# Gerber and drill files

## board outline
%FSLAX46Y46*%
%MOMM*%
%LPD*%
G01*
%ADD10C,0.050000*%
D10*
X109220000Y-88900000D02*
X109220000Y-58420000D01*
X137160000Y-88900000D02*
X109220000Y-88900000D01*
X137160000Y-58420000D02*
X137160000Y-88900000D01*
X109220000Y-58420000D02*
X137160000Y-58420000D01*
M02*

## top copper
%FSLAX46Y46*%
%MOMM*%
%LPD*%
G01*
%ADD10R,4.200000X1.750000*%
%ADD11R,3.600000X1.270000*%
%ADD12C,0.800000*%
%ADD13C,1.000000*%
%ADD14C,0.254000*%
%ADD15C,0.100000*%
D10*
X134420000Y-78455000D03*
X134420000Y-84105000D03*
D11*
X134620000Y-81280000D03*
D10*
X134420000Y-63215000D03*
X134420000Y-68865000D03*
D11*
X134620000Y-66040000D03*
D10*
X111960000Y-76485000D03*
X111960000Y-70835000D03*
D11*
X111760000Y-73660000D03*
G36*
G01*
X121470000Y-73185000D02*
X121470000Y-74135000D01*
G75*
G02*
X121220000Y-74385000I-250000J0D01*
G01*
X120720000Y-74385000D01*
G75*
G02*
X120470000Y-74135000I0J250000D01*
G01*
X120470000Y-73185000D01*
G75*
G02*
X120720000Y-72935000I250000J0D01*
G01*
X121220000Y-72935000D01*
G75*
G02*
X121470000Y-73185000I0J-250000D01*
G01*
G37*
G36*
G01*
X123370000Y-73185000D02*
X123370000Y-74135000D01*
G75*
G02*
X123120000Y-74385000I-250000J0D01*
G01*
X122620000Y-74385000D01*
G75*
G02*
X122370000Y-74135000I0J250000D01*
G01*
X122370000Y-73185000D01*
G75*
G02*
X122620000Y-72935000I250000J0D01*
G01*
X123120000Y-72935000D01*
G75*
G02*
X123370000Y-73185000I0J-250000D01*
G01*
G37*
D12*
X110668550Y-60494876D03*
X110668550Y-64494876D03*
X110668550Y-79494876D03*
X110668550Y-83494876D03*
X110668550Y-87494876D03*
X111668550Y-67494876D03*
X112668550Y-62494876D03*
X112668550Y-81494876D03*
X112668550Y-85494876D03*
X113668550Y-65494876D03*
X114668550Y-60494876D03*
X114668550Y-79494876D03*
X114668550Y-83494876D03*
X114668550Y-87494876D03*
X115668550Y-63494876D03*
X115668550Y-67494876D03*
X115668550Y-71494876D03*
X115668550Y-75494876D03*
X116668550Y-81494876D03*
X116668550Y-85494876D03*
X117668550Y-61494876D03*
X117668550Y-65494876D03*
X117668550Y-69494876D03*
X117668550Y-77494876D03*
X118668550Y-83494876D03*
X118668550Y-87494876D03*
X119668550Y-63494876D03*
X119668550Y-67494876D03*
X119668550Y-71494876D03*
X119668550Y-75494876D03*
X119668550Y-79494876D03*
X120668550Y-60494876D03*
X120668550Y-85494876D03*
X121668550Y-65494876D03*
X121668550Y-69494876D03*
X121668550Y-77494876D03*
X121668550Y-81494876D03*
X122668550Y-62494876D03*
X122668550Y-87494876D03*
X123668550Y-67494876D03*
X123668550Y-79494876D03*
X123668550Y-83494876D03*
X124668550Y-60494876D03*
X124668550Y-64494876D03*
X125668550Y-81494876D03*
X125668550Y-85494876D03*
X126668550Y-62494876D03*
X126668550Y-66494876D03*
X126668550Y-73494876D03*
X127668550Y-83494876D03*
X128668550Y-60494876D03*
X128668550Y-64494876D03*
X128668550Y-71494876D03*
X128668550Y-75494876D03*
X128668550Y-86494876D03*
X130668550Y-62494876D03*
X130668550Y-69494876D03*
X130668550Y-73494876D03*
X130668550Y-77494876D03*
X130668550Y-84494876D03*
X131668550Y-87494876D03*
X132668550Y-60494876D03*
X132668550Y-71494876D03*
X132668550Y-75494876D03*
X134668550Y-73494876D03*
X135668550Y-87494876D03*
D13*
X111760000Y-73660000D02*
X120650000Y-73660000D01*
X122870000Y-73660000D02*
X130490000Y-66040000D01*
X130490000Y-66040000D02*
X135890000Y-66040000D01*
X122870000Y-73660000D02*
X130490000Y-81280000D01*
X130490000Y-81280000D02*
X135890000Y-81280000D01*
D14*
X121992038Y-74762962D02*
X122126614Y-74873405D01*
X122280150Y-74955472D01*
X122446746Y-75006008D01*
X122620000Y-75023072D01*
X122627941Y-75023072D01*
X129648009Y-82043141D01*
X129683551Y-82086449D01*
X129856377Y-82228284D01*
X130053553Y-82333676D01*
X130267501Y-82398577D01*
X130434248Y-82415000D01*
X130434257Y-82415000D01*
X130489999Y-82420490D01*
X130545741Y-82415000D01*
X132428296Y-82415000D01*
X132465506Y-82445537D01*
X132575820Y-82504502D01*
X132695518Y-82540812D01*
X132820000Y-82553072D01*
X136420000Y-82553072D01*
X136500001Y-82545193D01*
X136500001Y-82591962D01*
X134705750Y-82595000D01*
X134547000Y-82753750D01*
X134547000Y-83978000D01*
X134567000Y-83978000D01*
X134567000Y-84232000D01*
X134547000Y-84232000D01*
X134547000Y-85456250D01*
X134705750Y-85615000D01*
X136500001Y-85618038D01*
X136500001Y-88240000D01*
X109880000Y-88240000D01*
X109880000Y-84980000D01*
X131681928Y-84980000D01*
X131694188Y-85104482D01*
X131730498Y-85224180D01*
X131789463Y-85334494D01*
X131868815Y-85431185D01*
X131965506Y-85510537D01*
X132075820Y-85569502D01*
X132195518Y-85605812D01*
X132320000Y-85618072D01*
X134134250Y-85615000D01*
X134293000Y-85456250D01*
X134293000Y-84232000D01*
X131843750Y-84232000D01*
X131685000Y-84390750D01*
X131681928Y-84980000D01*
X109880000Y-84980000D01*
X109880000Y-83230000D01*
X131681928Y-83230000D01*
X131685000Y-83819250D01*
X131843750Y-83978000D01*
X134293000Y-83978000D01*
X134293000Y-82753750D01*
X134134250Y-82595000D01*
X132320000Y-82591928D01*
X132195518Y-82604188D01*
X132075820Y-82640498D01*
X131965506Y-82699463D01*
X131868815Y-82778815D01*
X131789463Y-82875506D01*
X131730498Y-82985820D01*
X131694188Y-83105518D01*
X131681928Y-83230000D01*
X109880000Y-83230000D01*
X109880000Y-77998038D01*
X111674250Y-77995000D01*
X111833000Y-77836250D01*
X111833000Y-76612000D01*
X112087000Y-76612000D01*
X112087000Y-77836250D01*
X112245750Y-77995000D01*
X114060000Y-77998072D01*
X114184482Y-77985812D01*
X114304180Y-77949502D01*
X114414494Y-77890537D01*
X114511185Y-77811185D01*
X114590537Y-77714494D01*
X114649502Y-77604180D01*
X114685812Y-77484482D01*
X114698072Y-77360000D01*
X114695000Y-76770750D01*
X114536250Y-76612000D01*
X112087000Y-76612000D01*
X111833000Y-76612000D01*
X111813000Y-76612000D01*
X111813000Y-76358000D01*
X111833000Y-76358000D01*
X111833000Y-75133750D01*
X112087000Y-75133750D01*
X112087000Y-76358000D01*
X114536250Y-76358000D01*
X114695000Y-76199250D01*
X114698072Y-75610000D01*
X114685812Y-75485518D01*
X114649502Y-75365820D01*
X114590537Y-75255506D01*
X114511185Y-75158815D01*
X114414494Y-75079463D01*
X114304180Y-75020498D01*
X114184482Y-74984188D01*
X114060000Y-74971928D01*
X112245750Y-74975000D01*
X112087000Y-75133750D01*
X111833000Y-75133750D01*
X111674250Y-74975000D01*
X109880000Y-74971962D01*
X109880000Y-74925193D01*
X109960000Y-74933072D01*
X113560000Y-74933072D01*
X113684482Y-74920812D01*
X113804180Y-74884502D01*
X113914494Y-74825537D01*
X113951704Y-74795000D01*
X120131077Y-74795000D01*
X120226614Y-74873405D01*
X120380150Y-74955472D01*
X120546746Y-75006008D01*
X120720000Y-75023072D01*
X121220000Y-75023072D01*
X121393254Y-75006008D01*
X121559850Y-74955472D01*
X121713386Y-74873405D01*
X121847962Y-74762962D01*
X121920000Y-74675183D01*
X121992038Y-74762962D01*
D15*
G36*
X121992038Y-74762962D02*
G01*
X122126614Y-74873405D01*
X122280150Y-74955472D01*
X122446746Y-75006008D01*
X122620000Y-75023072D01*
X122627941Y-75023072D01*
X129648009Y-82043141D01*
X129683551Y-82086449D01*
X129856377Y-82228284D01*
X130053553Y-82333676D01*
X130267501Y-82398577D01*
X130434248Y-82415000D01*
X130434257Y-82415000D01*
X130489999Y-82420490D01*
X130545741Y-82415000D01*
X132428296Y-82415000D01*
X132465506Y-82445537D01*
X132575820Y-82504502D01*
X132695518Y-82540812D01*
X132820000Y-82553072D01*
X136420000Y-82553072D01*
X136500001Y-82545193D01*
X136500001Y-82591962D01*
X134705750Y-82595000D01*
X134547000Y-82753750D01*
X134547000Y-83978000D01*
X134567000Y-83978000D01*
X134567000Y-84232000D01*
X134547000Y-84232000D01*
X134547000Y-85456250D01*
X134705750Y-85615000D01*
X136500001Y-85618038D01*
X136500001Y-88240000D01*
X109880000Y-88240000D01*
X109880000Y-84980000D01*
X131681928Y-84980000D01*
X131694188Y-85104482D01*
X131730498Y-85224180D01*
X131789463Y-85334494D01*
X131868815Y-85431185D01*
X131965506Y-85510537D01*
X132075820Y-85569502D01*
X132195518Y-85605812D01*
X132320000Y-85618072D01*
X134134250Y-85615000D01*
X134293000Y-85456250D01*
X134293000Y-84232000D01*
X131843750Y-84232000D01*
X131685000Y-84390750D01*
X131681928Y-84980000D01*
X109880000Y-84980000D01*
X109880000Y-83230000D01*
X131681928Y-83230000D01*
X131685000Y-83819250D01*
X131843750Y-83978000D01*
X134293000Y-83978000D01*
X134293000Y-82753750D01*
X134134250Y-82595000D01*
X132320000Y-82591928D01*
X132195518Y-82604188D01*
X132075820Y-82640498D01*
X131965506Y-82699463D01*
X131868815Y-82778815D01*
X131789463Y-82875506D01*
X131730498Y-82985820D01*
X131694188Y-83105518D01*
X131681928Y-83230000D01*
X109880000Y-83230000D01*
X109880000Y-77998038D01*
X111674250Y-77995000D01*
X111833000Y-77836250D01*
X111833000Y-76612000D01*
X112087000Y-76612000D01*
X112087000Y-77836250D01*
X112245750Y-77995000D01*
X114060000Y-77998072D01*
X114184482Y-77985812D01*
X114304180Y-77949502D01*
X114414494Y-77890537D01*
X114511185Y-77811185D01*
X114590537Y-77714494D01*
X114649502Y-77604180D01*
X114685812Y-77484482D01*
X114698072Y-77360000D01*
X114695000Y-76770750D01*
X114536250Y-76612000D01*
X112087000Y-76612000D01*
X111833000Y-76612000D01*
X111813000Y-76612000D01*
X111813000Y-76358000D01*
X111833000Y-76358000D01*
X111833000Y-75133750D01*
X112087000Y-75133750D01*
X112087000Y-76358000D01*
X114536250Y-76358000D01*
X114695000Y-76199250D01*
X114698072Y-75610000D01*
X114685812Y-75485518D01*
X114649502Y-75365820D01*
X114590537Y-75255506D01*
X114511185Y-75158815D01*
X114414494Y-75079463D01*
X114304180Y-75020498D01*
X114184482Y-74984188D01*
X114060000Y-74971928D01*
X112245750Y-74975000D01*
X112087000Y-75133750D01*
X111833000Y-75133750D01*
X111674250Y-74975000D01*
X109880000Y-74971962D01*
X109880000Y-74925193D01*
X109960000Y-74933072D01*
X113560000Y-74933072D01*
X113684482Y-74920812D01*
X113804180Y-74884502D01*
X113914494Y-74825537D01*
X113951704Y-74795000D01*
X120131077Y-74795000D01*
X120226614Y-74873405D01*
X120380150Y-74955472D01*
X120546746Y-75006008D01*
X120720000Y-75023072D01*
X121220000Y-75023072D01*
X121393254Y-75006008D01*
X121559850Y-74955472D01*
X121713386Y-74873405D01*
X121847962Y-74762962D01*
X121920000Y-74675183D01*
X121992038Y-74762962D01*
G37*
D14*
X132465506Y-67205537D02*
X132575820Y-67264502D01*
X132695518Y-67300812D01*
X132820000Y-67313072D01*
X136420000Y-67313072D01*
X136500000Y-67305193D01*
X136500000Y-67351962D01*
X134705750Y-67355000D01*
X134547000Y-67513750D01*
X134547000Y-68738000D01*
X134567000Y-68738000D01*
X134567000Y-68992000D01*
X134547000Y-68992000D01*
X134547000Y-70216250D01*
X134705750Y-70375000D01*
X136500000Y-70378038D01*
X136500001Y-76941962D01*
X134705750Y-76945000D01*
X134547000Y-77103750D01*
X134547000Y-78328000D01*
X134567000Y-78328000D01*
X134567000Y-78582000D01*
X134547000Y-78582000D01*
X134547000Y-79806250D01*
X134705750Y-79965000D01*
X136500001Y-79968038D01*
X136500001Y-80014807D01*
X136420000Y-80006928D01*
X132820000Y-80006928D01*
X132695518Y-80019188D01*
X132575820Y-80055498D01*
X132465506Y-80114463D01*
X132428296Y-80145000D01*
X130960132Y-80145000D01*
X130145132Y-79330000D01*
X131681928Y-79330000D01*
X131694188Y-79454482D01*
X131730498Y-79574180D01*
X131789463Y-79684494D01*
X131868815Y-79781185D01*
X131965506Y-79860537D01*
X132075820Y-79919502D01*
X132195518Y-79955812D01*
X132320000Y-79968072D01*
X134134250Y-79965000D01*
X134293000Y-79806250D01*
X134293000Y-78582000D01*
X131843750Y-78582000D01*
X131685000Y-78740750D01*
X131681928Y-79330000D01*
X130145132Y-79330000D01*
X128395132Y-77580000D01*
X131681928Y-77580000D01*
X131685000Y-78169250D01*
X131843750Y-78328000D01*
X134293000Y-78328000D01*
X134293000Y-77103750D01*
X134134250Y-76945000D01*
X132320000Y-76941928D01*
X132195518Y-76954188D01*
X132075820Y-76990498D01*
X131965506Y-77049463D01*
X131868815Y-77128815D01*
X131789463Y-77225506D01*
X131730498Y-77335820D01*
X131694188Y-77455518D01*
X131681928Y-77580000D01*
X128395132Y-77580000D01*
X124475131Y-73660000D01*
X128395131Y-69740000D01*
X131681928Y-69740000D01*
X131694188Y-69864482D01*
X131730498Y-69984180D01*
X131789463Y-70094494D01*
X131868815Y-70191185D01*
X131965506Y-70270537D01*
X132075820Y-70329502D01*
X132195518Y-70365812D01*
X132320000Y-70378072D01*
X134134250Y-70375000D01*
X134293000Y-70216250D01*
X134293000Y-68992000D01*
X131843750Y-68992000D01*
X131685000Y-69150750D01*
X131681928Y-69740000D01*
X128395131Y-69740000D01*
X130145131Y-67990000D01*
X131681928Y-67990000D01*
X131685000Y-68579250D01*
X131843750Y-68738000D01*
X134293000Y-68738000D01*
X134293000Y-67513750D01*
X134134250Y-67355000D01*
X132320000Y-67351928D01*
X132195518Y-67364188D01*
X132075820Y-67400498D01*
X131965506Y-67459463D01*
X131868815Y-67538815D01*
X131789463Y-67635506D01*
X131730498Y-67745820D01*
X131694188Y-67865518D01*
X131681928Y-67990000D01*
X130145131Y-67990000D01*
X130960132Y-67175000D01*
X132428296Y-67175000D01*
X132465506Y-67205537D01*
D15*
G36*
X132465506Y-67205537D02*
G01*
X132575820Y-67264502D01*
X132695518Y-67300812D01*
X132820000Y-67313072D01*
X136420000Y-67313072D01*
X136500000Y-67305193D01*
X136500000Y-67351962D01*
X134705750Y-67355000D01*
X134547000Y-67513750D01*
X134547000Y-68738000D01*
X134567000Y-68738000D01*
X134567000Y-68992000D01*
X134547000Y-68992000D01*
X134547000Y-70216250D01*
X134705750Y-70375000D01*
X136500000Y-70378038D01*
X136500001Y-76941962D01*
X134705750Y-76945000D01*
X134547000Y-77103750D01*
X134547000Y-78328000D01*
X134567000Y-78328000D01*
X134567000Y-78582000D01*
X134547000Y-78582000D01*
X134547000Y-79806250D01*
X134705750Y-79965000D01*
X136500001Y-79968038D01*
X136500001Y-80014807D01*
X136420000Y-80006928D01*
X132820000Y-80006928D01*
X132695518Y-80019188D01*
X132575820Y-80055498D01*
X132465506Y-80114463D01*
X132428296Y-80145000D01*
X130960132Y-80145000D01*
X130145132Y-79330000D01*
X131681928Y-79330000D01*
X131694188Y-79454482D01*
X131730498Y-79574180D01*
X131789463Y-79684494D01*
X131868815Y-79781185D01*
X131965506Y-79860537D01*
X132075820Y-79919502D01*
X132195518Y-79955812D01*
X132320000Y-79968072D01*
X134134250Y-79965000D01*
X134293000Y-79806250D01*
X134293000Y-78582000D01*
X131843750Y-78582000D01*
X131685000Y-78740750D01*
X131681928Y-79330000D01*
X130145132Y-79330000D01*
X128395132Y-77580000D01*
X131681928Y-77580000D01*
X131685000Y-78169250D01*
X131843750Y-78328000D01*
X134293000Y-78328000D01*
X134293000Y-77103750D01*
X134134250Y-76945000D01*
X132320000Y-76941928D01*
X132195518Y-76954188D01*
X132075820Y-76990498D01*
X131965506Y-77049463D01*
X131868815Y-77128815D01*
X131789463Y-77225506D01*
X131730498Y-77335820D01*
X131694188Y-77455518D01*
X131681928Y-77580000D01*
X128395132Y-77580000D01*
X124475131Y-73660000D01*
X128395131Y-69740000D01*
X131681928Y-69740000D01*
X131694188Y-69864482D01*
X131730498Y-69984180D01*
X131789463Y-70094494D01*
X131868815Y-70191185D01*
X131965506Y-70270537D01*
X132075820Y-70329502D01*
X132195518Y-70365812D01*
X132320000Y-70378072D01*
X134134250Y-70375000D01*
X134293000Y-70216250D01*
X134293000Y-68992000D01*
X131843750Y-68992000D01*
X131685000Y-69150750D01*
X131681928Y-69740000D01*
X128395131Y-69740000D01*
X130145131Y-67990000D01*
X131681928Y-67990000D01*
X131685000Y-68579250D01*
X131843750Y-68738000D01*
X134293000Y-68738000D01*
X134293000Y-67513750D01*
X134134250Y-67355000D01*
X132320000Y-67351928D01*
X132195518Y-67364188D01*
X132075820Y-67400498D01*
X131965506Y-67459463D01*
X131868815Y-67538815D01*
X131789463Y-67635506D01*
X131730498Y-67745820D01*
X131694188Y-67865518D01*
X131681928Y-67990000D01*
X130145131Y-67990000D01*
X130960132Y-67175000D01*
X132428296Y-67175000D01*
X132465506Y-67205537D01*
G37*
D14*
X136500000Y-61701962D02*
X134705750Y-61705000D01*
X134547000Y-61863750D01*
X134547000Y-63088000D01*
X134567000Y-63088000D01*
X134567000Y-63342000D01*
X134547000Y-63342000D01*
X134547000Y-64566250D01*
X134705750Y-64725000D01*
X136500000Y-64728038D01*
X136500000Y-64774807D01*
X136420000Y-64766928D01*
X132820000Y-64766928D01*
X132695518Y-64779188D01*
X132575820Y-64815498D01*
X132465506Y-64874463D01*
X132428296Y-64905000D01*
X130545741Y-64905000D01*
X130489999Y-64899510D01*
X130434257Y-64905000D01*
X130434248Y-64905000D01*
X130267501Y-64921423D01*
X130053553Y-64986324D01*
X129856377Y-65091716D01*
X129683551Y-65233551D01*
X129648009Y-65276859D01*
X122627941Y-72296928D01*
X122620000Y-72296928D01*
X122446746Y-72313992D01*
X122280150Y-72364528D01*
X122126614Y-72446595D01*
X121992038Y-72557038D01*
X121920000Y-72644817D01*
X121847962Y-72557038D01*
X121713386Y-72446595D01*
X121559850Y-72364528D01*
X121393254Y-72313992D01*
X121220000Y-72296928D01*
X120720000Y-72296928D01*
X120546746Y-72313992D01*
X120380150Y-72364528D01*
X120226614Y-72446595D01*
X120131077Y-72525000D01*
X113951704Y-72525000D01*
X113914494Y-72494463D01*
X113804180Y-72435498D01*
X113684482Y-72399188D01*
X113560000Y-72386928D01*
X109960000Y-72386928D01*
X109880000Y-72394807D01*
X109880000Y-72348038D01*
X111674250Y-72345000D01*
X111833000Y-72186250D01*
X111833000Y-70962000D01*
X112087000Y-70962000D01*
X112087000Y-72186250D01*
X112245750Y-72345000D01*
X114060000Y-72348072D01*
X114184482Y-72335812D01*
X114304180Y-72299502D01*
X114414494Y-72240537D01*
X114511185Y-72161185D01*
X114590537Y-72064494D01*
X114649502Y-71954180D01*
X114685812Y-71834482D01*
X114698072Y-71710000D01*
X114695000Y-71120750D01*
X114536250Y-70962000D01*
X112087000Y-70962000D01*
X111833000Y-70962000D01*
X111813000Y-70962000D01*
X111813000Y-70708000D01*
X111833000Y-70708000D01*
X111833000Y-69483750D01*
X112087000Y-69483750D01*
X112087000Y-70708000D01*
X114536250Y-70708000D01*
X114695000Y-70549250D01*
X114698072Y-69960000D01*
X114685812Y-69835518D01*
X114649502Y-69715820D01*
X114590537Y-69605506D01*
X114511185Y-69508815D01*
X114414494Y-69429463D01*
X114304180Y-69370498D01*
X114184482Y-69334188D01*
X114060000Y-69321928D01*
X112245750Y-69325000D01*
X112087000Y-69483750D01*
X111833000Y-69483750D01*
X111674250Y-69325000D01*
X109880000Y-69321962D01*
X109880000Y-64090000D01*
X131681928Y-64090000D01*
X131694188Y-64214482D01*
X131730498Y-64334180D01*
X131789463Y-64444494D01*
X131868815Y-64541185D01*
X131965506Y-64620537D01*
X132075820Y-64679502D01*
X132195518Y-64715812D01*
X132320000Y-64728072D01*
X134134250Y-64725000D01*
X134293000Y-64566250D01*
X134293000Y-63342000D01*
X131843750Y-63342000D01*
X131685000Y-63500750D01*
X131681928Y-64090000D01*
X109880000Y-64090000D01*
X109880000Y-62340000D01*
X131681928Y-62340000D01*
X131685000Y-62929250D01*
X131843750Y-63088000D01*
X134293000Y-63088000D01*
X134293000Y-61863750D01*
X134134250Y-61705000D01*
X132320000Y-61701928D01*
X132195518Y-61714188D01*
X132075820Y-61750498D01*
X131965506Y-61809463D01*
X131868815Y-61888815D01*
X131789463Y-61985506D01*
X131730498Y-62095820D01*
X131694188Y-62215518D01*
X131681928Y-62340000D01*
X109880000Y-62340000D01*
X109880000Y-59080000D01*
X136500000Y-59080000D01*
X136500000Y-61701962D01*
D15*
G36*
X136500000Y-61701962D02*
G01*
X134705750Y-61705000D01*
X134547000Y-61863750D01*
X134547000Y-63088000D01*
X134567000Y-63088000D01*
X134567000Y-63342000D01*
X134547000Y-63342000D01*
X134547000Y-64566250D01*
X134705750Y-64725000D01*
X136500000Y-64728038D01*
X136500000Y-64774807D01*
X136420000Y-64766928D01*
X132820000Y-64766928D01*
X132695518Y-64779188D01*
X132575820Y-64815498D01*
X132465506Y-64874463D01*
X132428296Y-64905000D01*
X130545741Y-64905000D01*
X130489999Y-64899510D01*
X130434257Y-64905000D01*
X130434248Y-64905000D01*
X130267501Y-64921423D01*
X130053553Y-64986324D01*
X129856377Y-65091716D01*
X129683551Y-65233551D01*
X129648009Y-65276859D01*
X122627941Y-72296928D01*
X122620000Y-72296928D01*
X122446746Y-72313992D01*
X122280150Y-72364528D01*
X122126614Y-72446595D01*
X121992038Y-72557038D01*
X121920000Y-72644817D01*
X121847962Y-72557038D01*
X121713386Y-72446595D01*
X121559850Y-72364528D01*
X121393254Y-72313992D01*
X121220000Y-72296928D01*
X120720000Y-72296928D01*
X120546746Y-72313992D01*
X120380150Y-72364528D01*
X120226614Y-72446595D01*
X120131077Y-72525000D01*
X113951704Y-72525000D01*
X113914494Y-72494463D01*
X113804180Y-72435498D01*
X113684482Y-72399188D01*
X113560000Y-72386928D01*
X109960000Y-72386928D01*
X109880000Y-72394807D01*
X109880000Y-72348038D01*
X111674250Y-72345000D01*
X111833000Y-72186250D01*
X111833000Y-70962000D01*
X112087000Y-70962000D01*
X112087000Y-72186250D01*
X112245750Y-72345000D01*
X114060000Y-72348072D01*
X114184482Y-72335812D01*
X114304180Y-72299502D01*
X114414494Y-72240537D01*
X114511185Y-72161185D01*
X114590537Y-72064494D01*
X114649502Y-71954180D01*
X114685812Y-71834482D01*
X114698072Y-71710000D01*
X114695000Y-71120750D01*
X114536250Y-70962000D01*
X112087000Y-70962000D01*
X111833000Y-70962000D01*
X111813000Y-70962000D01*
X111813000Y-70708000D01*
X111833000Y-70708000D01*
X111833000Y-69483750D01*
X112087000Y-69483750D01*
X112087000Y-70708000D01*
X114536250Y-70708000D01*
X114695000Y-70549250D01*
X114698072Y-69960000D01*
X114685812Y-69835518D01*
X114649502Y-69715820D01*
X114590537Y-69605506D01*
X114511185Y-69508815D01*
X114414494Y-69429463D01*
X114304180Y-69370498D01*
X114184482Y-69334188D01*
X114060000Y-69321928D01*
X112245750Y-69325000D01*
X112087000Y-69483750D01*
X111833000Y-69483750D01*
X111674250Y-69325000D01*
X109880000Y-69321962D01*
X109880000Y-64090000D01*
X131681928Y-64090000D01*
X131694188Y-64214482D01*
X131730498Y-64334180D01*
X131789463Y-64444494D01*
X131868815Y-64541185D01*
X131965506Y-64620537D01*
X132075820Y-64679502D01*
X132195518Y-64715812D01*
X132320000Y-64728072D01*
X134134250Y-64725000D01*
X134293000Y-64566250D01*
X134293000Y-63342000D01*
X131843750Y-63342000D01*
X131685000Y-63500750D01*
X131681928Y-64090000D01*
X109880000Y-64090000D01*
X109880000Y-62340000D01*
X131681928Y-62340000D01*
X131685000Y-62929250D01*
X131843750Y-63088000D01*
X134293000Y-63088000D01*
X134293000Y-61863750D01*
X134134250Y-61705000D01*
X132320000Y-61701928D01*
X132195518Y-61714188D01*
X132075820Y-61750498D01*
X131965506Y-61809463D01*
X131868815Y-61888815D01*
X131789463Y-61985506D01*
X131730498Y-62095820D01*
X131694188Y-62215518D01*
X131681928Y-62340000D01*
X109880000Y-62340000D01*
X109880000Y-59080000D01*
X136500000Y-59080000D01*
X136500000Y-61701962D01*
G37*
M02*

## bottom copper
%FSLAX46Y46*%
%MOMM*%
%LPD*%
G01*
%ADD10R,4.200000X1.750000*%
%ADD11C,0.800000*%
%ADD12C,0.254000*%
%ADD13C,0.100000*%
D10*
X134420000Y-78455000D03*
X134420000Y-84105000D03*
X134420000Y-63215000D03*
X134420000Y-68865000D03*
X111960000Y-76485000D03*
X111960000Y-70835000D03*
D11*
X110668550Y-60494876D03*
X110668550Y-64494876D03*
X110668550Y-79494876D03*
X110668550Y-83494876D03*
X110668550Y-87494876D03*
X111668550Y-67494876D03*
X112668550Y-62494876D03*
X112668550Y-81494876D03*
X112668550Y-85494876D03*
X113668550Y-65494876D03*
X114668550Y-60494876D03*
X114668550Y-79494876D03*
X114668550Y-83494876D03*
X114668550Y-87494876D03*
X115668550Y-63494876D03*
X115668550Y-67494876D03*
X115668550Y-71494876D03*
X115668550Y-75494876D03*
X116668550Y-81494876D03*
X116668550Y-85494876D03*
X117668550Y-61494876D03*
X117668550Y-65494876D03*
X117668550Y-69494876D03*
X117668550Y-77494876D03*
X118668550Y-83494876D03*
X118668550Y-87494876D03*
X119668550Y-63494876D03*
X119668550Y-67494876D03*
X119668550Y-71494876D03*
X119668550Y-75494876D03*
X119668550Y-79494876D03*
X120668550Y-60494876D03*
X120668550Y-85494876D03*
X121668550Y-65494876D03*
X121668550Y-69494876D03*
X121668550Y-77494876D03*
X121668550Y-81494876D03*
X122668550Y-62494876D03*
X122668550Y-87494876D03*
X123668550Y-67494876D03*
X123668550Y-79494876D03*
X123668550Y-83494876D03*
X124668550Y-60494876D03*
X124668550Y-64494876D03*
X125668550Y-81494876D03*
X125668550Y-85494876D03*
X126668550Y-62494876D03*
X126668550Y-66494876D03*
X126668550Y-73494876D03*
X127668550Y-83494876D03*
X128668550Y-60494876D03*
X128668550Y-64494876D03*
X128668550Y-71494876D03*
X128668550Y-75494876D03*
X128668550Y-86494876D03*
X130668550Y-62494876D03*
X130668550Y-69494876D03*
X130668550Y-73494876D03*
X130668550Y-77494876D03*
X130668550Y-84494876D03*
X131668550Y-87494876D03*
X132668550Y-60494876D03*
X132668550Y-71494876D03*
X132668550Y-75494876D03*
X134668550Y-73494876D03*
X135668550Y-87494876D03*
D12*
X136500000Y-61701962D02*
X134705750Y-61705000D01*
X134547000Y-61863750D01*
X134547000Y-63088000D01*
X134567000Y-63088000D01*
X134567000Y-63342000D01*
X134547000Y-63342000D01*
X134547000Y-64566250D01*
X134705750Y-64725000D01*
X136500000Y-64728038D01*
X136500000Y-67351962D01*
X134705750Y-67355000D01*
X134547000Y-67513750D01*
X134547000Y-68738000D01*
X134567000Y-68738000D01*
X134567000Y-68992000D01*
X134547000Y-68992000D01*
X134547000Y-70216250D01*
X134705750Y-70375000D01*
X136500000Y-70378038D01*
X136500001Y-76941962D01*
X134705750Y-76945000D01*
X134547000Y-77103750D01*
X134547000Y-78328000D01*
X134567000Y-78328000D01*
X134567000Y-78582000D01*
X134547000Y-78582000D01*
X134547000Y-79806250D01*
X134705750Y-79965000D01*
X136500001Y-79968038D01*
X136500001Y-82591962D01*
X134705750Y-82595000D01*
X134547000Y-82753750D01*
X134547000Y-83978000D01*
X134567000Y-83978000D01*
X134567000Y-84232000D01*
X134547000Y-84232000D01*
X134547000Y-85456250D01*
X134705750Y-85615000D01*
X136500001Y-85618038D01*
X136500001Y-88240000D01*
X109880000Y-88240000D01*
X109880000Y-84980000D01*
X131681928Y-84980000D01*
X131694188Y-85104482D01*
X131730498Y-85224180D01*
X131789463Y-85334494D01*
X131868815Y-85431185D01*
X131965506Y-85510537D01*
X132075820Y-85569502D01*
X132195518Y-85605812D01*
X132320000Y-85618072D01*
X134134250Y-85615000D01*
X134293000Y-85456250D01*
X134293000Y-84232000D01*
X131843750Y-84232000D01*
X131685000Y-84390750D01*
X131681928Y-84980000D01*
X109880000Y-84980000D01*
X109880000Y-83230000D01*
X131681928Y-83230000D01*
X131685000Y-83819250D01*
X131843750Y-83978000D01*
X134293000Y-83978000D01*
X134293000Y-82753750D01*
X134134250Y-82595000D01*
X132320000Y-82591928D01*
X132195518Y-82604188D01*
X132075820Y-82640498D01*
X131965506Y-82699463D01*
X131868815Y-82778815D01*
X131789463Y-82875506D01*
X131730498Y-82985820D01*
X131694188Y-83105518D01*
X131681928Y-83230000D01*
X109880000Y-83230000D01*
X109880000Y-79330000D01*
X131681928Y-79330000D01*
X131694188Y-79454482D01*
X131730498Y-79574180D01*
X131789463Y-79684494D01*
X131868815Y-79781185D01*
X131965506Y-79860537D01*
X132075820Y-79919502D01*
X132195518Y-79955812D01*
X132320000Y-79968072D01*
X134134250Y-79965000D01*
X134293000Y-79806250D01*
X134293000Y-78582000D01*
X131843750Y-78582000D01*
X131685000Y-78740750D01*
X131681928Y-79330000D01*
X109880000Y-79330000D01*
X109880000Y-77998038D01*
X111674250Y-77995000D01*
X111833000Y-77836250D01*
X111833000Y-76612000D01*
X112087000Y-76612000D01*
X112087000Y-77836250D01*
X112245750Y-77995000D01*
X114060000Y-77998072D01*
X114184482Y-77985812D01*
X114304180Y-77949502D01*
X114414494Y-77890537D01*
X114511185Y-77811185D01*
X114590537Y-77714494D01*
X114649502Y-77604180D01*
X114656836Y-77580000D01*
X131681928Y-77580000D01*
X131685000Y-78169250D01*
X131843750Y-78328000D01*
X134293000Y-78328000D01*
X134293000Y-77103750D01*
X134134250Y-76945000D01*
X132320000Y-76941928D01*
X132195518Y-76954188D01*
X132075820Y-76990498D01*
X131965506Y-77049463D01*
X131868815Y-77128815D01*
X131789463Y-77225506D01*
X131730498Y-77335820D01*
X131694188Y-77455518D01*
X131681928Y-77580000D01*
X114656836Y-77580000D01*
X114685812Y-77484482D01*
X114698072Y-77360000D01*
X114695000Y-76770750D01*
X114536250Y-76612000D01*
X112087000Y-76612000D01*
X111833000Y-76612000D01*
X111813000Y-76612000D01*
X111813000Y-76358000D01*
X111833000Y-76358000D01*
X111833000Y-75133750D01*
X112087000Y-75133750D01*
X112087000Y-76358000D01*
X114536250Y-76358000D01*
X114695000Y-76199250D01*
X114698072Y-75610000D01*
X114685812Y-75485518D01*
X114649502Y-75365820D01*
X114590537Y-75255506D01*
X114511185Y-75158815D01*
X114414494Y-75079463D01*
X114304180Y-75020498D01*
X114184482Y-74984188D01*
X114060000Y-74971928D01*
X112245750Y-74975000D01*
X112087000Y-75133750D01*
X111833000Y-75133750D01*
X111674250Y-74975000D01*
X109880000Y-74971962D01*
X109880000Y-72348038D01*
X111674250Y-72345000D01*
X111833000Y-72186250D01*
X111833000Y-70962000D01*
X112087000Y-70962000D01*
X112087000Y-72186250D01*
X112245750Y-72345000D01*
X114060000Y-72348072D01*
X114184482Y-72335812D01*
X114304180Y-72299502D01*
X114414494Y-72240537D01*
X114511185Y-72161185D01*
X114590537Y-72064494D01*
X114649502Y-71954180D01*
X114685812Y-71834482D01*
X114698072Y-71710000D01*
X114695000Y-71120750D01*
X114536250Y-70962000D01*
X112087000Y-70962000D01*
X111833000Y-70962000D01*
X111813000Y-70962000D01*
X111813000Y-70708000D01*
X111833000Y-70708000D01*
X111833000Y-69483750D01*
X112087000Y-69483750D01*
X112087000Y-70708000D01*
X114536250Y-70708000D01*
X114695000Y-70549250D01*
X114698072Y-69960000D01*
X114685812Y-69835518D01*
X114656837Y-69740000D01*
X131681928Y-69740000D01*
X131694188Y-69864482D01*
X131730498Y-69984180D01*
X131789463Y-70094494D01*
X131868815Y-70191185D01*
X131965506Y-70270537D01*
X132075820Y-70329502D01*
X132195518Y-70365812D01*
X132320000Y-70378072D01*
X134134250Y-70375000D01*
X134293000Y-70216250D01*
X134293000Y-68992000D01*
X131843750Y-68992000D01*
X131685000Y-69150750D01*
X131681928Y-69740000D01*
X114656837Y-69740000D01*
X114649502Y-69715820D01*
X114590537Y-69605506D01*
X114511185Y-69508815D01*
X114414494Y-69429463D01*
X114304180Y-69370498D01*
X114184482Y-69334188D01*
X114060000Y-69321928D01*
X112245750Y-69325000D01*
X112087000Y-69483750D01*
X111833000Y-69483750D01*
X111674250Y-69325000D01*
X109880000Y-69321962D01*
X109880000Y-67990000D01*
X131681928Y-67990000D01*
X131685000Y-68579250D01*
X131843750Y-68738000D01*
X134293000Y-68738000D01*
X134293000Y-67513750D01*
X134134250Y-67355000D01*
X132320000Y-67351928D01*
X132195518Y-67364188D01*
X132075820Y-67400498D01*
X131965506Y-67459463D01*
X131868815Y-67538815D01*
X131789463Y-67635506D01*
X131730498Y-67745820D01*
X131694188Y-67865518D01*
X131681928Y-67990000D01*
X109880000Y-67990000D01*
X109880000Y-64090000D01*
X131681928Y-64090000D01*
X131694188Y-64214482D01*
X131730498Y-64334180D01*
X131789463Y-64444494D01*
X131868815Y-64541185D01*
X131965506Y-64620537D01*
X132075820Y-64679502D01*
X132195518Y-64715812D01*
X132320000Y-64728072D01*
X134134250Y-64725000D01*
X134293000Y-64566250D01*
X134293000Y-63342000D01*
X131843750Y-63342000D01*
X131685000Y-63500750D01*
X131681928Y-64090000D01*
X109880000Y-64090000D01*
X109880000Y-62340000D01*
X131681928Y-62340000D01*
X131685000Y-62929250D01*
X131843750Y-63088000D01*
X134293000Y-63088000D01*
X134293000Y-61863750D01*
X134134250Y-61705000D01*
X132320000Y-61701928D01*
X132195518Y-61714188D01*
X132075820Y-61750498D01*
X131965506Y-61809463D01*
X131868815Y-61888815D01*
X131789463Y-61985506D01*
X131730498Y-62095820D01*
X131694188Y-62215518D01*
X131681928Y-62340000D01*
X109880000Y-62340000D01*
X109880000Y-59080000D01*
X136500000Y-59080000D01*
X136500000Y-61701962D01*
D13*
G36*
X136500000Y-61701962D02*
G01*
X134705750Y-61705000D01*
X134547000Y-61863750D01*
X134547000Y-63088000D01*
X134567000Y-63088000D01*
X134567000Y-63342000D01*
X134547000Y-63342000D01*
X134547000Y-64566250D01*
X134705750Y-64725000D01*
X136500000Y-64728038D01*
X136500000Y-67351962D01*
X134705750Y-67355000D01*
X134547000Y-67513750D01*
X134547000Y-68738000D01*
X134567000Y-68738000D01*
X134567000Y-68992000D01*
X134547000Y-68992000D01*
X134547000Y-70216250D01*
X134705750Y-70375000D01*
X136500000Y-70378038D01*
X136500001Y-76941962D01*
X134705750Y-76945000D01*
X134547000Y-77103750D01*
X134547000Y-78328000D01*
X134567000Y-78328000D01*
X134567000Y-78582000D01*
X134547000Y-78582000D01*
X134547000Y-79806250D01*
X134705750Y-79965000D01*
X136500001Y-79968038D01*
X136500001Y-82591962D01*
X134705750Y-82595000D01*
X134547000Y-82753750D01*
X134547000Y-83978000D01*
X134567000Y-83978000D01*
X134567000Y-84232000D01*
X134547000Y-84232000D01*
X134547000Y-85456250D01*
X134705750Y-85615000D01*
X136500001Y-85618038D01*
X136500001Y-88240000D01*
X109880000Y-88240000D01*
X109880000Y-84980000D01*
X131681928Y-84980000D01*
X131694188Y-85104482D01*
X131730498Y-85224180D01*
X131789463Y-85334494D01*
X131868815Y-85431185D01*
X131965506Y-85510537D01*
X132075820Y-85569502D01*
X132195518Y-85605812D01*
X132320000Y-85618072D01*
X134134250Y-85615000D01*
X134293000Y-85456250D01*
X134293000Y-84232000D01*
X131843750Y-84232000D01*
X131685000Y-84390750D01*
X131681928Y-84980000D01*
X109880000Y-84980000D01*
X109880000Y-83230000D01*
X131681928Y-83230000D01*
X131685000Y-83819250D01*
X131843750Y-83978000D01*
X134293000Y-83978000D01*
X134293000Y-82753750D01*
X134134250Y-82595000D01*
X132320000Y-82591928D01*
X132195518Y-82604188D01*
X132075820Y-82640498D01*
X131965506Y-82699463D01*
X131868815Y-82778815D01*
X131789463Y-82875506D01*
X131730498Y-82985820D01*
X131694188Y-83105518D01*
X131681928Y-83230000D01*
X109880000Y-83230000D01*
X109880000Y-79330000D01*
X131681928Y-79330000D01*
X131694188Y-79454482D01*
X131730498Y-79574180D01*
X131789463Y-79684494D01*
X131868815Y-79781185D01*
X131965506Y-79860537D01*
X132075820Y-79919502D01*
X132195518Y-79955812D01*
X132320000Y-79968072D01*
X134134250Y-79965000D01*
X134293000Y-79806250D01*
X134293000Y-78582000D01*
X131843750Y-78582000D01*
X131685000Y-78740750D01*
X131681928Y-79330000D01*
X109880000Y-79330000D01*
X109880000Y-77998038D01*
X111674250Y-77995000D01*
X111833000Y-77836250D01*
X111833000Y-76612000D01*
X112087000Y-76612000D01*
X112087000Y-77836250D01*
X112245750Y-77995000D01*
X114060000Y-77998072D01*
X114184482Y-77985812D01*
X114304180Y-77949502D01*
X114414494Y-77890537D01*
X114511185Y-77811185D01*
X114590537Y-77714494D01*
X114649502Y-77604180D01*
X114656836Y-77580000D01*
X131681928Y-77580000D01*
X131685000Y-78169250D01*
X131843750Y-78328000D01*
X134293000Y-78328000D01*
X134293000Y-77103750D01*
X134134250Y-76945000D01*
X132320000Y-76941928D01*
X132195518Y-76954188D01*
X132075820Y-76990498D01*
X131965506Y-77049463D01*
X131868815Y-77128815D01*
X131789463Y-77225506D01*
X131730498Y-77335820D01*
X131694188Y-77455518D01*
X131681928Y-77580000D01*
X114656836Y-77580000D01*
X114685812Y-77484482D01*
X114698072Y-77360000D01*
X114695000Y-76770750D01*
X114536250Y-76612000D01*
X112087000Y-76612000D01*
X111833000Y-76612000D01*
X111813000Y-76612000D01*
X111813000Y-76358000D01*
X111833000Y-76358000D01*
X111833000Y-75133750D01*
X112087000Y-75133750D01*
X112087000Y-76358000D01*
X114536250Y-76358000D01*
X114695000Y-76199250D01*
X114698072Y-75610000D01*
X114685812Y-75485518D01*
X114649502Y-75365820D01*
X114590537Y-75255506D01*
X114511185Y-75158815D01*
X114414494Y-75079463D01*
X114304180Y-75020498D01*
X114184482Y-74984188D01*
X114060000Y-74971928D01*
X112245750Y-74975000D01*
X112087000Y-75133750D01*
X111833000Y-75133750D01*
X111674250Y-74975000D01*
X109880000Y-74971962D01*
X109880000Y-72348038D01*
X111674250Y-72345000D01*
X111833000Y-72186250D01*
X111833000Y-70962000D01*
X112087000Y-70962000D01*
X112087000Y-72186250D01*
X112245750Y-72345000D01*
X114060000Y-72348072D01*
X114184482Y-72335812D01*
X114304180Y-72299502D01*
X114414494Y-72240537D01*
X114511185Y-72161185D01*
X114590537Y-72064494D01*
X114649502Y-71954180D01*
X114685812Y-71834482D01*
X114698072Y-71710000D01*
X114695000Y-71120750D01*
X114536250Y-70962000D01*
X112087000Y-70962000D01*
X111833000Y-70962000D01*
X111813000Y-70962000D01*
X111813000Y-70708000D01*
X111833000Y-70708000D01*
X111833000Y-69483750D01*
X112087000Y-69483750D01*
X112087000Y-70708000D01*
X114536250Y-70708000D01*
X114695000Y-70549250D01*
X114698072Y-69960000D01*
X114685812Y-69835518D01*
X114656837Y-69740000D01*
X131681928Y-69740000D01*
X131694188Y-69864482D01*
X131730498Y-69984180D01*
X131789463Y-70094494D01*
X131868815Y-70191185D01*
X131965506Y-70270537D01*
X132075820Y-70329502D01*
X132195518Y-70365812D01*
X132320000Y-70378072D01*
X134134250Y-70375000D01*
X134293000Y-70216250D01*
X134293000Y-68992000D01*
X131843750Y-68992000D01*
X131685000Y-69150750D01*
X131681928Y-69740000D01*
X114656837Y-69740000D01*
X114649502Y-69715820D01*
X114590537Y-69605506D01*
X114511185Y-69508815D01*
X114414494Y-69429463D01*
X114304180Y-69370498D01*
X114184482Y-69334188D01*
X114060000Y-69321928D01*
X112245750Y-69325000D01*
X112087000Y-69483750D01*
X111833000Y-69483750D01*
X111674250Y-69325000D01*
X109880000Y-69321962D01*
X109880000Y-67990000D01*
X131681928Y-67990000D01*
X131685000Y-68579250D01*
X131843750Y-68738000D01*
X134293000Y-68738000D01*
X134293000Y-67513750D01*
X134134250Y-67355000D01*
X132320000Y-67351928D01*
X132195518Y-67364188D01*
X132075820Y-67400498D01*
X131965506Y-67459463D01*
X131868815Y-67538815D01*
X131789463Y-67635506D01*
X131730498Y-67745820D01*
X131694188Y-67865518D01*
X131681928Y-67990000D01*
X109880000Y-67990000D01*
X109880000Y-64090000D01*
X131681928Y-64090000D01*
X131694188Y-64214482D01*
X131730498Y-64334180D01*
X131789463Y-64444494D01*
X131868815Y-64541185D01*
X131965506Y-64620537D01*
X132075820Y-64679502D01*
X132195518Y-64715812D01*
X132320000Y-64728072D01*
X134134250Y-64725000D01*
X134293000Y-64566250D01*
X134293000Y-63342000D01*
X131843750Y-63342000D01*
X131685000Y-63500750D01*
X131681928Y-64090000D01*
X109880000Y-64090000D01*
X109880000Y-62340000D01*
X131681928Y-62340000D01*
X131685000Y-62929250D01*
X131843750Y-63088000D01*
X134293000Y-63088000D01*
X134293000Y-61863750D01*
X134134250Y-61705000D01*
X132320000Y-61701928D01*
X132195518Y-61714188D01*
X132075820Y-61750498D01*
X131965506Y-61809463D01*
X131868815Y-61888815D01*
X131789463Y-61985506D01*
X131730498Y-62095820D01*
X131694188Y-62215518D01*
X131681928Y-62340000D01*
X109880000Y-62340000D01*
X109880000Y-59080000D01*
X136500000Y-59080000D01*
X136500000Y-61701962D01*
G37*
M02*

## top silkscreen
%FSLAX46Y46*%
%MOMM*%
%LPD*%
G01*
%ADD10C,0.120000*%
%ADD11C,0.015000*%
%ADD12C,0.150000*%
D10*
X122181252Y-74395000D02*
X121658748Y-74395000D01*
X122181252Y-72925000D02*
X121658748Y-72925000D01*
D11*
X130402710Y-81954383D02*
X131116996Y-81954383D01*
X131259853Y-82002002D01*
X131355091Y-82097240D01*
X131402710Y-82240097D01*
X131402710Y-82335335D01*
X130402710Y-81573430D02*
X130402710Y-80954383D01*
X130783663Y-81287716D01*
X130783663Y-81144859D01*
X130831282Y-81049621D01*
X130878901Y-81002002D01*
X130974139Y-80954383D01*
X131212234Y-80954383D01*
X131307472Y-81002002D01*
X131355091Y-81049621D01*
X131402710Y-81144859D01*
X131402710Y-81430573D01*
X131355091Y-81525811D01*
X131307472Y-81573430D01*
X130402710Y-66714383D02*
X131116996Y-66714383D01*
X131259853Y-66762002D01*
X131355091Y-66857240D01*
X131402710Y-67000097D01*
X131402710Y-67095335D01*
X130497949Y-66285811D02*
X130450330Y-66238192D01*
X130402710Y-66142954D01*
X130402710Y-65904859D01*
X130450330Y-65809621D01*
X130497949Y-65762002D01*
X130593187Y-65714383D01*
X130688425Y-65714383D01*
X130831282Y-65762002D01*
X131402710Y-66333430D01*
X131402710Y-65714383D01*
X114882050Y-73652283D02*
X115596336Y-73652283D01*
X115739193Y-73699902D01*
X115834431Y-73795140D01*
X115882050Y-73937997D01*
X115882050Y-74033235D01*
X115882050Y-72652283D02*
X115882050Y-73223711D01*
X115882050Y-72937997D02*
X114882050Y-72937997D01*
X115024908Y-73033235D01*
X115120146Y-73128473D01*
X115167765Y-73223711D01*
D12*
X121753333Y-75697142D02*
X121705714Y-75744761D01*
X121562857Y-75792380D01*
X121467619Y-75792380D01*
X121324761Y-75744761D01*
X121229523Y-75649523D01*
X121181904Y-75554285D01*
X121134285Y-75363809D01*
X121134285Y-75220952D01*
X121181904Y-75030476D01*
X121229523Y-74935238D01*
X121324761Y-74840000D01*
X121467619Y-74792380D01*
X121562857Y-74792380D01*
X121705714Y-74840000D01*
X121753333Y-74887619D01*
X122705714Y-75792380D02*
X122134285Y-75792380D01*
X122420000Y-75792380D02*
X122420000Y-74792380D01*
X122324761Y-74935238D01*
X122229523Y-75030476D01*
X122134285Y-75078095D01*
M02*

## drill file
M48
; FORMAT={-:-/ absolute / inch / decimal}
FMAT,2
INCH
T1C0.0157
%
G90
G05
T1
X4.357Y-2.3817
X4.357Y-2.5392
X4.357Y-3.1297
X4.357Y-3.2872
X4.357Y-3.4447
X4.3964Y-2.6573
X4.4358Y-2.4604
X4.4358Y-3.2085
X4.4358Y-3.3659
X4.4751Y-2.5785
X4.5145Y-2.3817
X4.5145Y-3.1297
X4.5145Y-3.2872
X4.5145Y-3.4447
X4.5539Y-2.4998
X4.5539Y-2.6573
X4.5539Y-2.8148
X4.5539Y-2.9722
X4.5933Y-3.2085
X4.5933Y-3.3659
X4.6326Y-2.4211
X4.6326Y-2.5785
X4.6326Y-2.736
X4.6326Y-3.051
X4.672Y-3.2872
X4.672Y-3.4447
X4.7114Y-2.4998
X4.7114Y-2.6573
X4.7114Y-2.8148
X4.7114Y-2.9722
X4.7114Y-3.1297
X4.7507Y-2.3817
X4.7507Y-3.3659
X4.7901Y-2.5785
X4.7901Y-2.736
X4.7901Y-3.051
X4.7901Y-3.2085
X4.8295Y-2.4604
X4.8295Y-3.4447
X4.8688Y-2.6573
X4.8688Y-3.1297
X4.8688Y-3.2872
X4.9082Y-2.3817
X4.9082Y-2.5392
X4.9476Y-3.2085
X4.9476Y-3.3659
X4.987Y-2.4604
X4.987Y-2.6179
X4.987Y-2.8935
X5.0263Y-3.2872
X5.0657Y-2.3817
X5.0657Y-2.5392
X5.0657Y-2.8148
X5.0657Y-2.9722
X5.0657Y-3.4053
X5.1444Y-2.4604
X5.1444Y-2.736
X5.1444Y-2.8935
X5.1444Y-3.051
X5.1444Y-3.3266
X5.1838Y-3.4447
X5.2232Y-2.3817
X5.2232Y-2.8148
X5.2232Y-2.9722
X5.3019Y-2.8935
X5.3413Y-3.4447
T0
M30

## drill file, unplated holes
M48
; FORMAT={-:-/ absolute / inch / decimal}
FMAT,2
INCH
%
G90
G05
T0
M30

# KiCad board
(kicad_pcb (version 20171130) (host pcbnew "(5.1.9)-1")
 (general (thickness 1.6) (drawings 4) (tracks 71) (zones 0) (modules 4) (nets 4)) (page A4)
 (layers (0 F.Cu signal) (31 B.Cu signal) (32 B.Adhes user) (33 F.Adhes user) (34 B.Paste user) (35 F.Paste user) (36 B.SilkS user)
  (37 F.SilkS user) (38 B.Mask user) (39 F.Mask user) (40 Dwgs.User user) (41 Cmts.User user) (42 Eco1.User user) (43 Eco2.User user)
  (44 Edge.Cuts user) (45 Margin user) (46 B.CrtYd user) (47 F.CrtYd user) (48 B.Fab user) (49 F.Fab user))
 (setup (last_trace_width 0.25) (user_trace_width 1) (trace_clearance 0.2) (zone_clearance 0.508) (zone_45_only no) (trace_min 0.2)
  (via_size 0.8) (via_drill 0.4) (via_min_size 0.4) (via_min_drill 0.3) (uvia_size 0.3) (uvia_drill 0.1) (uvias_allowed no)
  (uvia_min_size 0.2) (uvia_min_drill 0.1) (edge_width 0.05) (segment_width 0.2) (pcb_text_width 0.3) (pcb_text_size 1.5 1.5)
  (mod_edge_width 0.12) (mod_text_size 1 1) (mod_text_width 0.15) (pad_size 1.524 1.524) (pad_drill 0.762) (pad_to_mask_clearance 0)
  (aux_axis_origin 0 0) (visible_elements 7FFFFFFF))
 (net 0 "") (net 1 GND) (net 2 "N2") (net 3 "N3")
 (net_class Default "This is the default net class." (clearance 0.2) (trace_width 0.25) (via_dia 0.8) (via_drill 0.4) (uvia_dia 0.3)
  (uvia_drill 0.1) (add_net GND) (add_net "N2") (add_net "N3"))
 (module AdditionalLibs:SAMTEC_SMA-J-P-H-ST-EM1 (layer F.Cu) (at 134.62 81.28 90)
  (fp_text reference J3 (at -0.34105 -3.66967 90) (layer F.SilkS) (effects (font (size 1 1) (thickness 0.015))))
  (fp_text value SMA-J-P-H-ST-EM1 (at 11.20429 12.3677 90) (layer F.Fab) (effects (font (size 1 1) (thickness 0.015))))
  (pad 3_2 smd rect (at 2.825 -0.2 90) (size 1.75 4.2) (layers B.Cu B.Paste B.Mask) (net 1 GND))
  (pad 2_2 smd rect (at -2.825 -0.2 90) (size 1.75 4.2) (layers B.Cu B.Paste B.Mask) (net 1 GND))
  (pad 3_1 smd rect (at 2.825 -0.2 90) (size 1.75 4.2) (layers F.Cu F.Paste F.Mask) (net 1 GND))
  (pad 2_1 smd rect (at -2.825 -0.2 90) (size 1.75 4.2) (layers F.Cu F.Paste F.Mask) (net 1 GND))
  (pad 1 smd rect (at 0 0 90) (size 1.27 3.6) (layers F.Cu F.Paste F.Mask) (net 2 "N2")))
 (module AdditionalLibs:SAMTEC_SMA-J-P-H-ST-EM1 (layer F.Cu) (at 134.62 66.04 90)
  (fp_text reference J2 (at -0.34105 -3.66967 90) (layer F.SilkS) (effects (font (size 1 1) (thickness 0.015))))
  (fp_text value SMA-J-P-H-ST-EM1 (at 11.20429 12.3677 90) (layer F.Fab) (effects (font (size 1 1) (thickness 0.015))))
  (pad 3_2 smd rect (at 2.825 -0.2 90) (size 1.75 4.2) (layers B.Cu B.Paste B.Mask) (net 1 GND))
  (pad 2_2 smd rect (at -2.825 -0.2 90) (size 1.75 4.2) (layers B.Cu B.Paste B.Mask) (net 1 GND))
  (pad 3_1 smd rect (at 2.825 -0.2 90) (size 1.75 4.2) (layers F.Cu F.Paste F.Mask) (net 1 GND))
  (pad 2_1 smd rect (at -2.825 -0.2 90) (size 1.75 4.2) (layers F.Cu F.Paste F.Mask) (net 1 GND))
  (pad 1 smd rect (at 0 0 90) (size 1.27 3.6) (layers F.Cu F.Paste F.Mask) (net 2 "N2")))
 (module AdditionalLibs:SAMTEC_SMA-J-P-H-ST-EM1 (layer F.Cu) (at 111.76 73.66 270)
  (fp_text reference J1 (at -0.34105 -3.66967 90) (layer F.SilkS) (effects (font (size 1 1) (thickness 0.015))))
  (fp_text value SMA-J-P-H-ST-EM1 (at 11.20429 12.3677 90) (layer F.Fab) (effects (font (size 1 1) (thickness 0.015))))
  (pad 3_2 smd rect (at 2.825 -0.2 270) (size 1.75 4.2) (layers B.Cu B.Paste B.Mask) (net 1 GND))
  (pad 2_2 smd rect (at -2.825 -0.2 270) (size 1.75 4.2) (layers B.Cu B.Paste B.Mask) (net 1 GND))
  (pad 3_1 smd rect (at 2.825 -0.2 270) (size 1.75 4.2) (layers F.Cu F.Paste F.Mask) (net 1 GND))
  (pad 2_1 smd rect (at -2.825 -0.2 270) (size 1.75 4.2) (layers F.Cu F.Paste F.Mask) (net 1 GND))
  (pad 1 smd rect (at 0 0 270) (size 1.27 3.6) (layers F.Cu F.Paste F.Mask) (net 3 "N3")))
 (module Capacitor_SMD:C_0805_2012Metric (layer F.Cu) (at 121.92 73.66 180)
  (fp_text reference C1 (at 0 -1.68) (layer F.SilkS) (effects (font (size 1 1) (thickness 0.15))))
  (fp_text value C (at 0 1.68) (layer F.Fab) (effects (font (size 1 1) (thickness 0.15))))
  (fp_line (start -0.261252 -0.735) (end 0.261252 -0.735) (layer F.SilkS) (width 0.12))
  (fp_line (start -0.261252 0.735) (end 0.261252 0.735) (layer F.SilkS) (width 0.12))
  (pad 2 smd roundrect (at 0.95 0 180) (size 1 1.45) (layers F.Cu F.Paste F.Mask) (roundrect_rratio 0.25) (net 3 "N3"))
  (pad 1 smd roundrect (at -0.95 0 180) (size 1 1.45) (layers F.Cu F.Paste F.Mask) (roundrect_rratio 0.25) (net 2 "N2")))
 (gr_line (start 109.22 88.9) (end 109.22 58.42) (layer Edge.Cuts) (width 0.05))
 (gr_line (start 137.16 88.9) (end 109.22 88.9) (layer Edge.Cuts) (width 0.05))
 (gr_line (start 137.16 58.42) (end 137.16 88.9) (layer Edge.Cuts) (width 0.05))
 (gr_line (start 109.22 58.42) (end 137.16 58.42) (layer Edge.Cuts) (width 0.05))
 (via (at 110.66855 60.494876) (size 0.8) (drill 0.4) (layers F.Cu B.Cu) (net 1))
 (via (at 110.66855 64.494876) (size 0.8) (drill 0.4) (layers F.Cu B.Cu) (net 1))
 (via (at 110.66855 79.494876) (size 0.8) (drill 0.4) (layers F.Cu B.Cu) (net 1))
 (via (at 110.66855 83.494876) (size 0.8) (drill 0.4) (layers F.Cu B.Cu) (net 1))
 (via (at 110.66855 87.494876) (size 0.8) (drill 0.4) (layers F.Cu B.Cu) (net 1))
 (via (at 111.66855 67.494876) (size 0.8) (drill 0.4) (layers F.Cu B.Cu) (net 1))
 (via (at 112.66855 62.494876) (size 0.8) (drill 0.4) (layers F.Cu B.Cu) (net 1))
 (via (at 112.66855 81.494876) (size 0.8) (drill 0.4) (layers F.Cu B.Cu) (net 1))
 (via (at 112.66855 85.494876) (size 0.8) (drill 0.4) (layers F.Cu B.Cu) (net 1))
 (via (at 113.66855 65.494876) (size 0.8) (drill 0.4) (layers F.Cu B.Cu) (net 1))
 (via (at 114.66855 60.494876) (size 0.8) (drill 0.4) (layers F.Cu B.Cu) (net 1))
 (via (at 114.66855 79.494876) (size 0.8) (drill 0.4) (layers F.Cu B.Cu) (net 1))
 (via (at 114.66855 83.494876) (size 0.8) (drill 0.4) (layers F.Cu B.Cu) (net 1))
 (via (at 114.66855 87.494876) (size 0.8) (drill 0.4) (layers F.Cu B.Cu) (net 1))
 (via (at 115.66855 63.494876) (size 0.8) (drill 0.4) (layers F.Cu B.Cu) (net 1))
 (via (at 115.66855 67.494876) (size 0.8) (drill 0.4) (layers F.Cu B.Cu) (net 1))
 (via (at 115.66855 71.494876) (size 0.8) (drill 0.4) (layers F.Cu B.Cu) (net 1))
 (via (at 115.66855 75.494876) (size 0.8) (drill 0.4) (layers F.Cu B.Cu) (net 1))
 (via (at 116.66855 81.494876) (size 0.8) (drill 0.4) (layers F.Cu B.Cu) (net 1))
 (via (at 116.66855 85.494876) (size 0.8) (drill 0.4) (layers F.Cu B.Cu) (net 1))
 (via (at 117.66855 61.494876) (size 0.8) (drill 0.4) (layers F.Cu B.Cu) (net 1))
 (via (at 117.66855 65.494876) (size 0.8) (drill 0.4) (layers F.Cu B.Cu) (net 1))
 (via (at 117.66855 69.494876) (size 0.8) (drill 0.4) (layers F.Cu B.Cu) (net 1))
 (via (at 117.66855 77.494876) (size 0.8) (drill 0.4) (layers F.Cu B.Cu) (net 1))
 (via (at 118.66855 83.494876) (size 0.8) (drill 0.4) (layers F.Cu B.Cu) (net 1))
 (via (at 118.66855 87.494876) (size 0.8) (drill 0.4) (layers F.Cu B.Cu) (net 1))
 (via (at 119.66855 63.494876) (size 0.8) (drill 0.4) (layers F.Cu B.Cu) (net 1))
 (via (at 119.66855 67.494876) (size 0.8) (drill 0.4) (layers F.Cu B.Cu) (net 1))
 (via (at 119.66855 71.494876) (size 0.8) (drill 0.4) (layers F.Cu B.Cu) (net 1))
 (via (at 119.66855 75.494876) (size 0.8) (drill 0.4) (layers F.Cu B.Cu) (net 1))
 (via (at 119.66855 79.494876) (size 0.8) (drill 0.4) (layers F.Cu B.Cu) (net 1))
 (via (at 120.66855 60.494876) (size 0.8) (drill 0.4) (layers F.Cu B.Cu) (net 1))
 (via (at 120.66855 85.494876) (size 0.8) (drill 0.4) (layers F.Cu B.Cu) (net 1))
 (via (at 121.66855 65.494876) (size 0.8) (drill 0.4) (layers F.Cu B.Cu) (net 1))
 (via (at 121.66855 69.494876) (size 0.8) (drill 0.4) (layers F.Cu B.Cu) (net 1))
 (via (at 121.66855 77.494876) (size 0.8) (drill 0.4) (layers F.Cu B.Cu) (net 1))
 (via (at 121.66855 81.494876) (size 0.8) (drill 0.4) (layers F.Cu B.Cu) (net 1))
 (via (at 122.66855 62.494876) (size 0.8) (drill 0.4) (layers F.Cu B.Cu) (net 1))
 (via (at 122.66855 87.494876) (size 0.8) (drill 0.4) (layers F.Cu B.Cu) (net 1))
 (via (at 123.66855 67.494876) (size 0.8) (drill 0.4) (layers F.Cu B.Cu) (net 1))
 (via (at 123.66855 79.494876) (size 0.8) (drill 0.4) (layers F.Cu B.Cu) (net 1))
 (via (at 123.66855 83.494876) (size 0.8) (drill 0.4) (layers F.Cu B.Cu) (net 1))
 (via (at 124.66855 60.494876) (size 0.8) (drill 0.4) (layers F.Cu B.Cu) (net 1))
 (via (at 124.66855 64.494876) (size 0.8) (drill 0.4) (layers F.Cu B.Cu) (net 1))
 (via (at 125.66855 81.494876) (size 0.8) (drill 0.4) (layers F.Cu B.Cu) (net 1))
 (via (at 125.66855 85.494876) (size 0.8) (drill 0.4) (layers F.Cu B.Cu) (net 1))
 (via (at 126.66855 62.494876) (size 0.8) (drill 0.4) (layers F.Cu B.Cu) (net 1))
 (via (at 126.66855 66.494876) (size 0.8) (drill 0.4) (layers F.Cu B.Cu) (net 1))
 (via (at 126.66855 73.494876) (size 0.8) (drill 0.4) (layers F.Cu B.Cu) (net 1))
 (via (at 127.66855 83.494876) (size 0.8) (drill 0.4) (layers F.Cu B.Cu) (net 1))
 (via (at 128.66855 60.494876) (size 0.8) (drill 0.4) (layers F.Cu B.Cu) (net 1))
 (via (at 128.66855 64.494876) (size 0.8) (drill 0.4) (layers F.Cu B.Cu) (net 1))
 (via (at 128.66855 71.494876) (size 0.8) (drill 0.4) (layers F.Cu B.Cu) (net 1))
 (via (at 128.66855 75.494876) (size 0.8) (drill 0.4) (layers F.Cu B.Cu) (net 1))
 (via (at 128.66855 86.494876) (size 0.8) (drill 0.4) (layers F.Cu B.Cu) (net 1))
 (via (at 130.66855 62.494876) (size 0.8) (drill 0.4) (layers F.Cu B.Cu) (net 1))
 (via (at 130.66855 69.494876) (size 0.8) (drill 0.4) (layers F.Cu B.Cu) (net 1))
 (via (at 130.66855 73.494876) (size 0.8) (drill 0.4) (layers F.Cu B.Cu) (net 1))
 (via (at 130.66855 77.494876) (size 0.8) (drill 0.4) (layers F.Cu B.Cu) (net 1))
 (via (at 130.66855 84.494876) (size 0.8) (drill 0.4) (layers F.Cu B.Cu) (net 1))
 (via (at 131.66855 87.494876) (size 0.8) (drill 0.4) (layers F.Cu B.Cu) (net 1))
 (via (at 132.66855 60.494876) (size 0.8) (drill 0.4) (layers F.Cu B.Cu) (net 1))
 (via (at 132.66855 71.494876) (size 0.8) (drill 0.4) (layers F.Cu B.Cu) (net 1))
 (via (at 132.66855 75.494876) (size 0.8) (drill 0.4) (layers F.Cu B.Cu) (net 1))
 (via (at 134.66855 73.494876) (size 0.8) (drill 0.4) (layers F.Cu B.Cu) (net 1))
 (via (at 135.66855 87.494876) (size 0.8) (drill 0.4) (layers F.Cu B.Cu) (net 1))
 (segment (start 111.76 73.66) (end 120.65 73.66) (width 1) (layer F.Cu) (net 3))
 (segment (start 122.87 73.66) (end 130.49 66.04) (width 1) (layer F.Cu) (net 2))
 (segment (start 130.49 66.04) (end 135.89 66.04) (width 1) (layer F.Cu) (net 2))
 (segment (start 122.87 73.66) (end 130.49 81.28) (width 1) (layer F.Cu) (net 2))
 (segment (start 130.49 81.28) (end 135.89 81.28) (width 1) (layer F.Cu) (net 2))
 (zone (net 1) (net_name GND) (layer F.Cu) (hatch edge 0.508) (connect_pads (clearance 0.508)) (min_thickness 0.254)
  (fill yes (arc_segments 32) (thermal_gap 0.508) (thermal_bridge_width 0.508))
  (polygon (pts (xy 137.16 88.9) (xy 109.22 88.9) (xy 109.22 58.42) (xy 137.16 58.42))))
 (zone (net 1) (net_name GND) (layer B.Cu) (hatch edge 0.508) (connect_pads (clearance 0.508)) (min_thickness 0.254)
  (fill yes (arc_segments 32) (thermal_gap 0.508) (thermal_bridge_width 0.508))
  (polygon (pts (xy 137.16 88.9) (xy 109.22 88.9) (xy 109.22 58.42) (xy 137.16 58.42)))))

